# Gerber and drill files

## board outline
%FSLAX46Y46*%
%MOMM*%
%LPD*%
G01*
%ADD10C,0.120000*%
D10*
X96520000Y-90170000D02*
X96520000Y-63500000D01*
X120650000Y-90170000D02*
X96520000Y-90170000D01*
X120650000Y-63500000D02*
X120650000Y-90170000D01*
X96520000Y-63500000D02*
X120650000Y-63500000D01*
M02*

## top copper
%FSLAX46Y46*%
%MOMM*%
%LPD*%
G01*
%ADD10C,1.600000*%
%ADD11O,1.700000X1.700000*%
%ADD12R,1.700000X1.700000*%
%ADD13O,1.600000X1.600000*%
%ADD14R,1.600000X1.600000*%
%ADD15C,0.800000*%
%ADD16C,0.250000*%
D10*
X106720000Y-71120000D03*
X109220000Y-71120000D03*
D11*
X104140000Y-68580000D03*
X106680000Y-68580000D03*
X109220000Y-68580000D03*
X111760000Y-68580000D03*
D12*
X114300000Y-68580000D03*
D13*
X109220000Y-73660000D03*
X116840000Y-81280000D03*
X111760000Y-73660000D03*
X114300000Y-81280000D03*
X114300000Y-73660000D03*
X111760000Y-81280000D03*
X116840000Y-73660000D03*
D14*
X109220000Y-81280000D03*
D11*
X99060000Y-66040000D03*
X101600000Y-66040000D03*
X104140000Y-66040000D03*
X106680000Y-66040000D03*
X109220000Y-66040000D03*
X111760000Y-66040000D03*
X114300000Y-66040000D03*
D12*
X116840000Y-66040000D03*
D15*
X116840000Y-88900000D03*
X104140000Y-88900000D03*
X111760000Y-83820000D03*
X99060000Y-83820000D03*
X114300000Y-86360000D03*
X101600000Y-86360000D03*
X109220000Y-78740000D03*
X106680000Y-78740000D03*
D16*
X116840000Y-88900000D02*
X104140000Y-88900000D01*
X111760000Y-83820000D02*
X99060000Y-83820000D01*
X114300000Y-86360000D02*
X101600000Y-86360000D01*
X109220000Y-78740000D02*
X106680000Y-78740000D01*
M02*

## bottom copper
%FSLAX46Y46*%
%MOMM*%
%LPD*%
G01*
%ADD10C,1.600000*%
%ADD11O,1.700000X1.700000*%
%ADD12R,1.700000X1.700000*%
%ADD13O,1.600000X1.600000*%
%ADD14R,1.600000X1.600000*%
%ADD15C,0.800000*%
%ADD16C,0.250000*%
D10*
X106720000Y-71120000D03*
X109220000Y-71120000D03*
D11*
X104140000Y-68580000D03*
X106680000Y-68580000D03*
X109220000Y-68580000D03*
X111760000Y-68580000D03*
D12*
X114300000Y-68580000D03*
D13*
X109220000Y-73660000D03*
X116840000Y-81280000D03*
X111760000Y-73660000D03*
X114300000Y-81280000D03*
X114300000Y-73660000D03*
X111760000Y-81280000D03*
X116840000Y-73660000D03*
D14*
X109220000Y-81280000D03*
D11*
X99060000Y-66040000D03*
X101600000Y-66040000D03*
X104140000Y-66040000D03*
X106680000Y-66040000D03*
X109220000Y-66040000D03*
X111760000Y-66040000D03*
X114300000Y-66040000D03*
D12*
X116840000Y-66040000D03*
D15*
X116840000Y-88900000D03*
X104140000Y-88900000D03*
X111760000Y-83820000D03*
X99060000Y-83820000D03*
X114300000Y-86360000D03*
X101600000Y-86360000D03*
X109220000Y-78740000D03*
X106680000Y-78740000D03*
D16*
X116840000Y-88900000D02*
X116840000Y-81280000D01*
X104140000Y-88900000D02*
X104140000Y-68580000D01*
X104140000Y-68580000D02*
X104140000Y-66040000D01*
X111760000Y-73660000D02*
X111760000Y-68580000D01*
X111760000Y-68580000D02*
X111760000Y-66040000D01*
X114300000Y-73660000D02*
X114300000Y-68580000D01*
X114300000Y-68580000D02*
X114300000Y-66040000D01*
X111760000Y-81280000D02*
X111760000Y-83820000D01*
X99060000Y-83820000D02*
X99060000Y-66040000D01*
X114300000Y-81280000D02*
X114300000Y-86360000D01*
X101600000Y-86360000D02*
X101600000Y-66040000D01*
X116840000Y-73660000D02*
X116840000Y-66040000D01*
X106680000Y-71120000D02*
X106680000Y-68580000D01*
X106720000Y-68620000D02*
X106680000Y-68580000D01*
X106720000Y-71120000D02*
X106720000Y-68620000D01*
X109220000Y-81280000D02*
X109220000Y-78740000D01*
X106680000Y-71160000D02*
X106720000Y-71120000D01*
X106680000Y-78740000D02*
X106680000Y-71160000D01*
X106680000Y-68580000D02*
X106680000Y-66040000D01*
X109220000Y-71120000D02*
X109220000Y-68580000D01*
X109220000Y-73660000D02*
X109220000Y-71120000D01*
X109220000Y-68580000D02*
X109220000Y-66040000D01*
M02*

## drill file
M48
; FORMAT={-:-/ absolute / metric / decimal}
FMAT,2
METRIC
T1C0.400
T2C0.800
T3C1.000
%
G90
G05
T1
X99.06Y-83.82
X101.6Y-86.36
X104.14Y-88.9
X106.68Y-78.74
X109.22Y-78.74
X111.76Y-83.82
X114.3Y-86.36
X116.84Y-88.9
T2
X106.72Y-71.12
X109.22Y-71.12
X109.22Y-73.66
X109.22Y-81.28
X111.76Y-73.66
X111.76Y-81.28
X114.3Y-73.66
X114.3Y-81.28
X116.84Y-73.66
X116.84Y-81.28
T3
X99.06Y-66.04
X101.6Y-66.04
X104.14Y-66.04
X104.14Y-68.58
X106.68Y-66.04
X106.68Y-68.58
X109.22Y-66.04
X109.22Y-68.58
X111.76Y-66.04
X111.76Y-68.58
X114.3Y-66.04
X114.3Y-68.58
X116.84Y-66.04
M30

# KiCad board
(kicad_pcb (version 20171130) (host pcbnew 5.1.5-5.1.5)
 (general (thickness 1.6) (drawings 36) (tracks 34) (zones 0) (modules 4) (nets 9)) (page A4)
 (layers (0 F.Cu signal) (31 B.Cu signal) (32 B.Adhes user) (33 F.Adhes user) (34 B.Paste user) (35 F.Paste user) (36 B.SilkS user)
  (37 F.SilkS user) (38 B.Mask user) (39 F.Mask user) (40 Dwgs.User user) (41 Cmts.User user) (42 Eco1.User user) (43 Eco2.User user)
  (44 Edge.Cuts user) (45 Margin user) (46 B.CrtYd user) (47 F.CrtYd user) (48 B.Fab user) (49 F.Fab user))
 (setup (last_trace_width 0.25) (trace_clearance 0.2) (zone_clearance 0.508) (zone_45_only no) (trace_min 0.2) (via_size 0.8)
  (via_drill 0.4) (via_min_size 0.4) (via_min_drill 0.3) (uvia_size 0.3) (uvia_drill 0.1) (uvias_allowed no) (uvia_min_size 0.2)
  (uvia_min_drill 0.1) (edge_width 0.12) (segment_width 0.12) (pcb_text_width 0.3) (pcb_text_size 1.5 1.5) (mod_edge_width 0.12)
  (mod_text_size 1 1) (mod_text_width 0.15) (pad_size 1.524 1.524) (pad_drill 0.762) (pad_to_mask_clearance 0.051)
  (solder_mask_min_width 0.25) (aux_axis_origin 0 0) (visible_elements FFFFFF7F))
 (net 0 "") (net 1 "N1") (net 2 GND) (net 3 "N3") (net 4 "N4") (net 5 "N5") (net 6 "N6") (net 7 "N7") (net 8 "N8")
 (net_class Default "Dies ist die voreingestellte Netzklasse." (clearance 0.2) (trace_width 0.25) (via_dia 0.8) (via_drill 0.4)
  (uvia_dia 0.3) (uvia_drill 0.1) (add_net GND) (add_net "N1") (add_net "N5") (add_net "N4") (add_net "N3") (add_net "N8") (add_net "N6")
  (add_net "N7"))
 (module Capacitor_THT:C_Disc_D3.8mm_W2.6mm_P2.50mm (layer F.Cu) (at 109.22 71.12 180)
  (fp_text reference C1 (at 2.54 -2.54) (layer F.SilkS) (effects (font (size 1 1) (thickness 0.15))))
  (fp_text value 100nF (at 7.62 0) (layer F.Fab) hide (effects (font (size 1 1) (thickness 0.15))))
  (pad 2 thru_hole circle (at 2.5 0 180) (size 1.6 1.6) (drill 0.8) (layers *.Cu *.Mask) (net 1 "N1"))
  (pad 1 thru_hole circle (at 0 0 180) (size 1.6 1.6) (drill 0.8) (layers *.Cu *.Mask) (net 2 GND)))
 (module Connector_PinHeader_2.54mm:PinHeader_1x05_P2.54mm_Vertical (layer F.Cu) (at 114.3 68.58 270)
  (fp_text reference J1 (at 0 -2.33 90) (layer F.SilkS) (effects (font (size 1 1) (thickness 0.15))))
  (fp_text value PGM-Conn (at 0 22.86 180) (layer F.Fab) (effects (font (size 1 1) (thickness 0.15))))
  (pad 5 thru_hole oval (at 0 10.16 270) (size 1.7 1.7) (drill 1) (layers *.Cu *.Mask) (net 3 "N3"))
  (pad 4 thru_hole oval (at 0 7.62 270) (size 1.7 1.7) (drill 1) (layers *.Cu *.Mask) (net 1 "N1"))
  (pad 3 thru_hole oval (at 0 5.08 270) (size 1.7 1.7) (drill 1) (layers *.Cu *.Mask) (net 2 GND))
  (pad 2 thru_hole oval (at 0 2.54 270) (size 1.7 1.7) (drill 1) (layers *.Cu *.Mask) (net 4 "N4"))
  (pad 1 thru_hole rect (at 0 0 270) (size 1.7 1.7) (drill 1) (layers *.Cu *.Mask) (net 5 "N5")))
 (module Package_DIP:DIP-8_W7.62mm (layer F.Cu) (at 109.22 81.28 90)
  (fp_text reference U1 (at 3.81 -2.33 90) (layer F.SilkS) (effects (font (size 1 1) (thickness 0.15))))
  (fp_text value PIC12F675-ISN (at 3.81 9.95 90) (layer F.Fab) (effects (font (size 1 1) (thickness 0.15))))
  (pad 8 thru_hole oval (at 7.62 0 90) (size 1.6 1.6) (drill 0.8) (layers *.Cu *.Mask) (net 2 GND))
  (pad 4 thru_hole oval (at 0 7.62 90) (size 1.6 1.6) (drill 0.8) (layers *.Cu *.Mask) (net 3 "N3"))
  (pad 7 thru_hole oval (at 7.62 2.54 90) (size 1.6 1.6) (drill 0.8) (layers *.Cu *.Mask) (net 4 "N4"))
  (pad 3 thru_hole oval (at 0 5.08 90) (size 1.6 1.6) (drill 0.8) (layers *.Cu *.Mask) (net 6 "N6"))
  (pad 6 thru_hole oval (at 7.62 5.08 90) (size 1.6 1.6) (drill 0.8) (layers *.Cu *.Mask) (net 5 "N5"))
  (pad 2 thru_hole oval (at 0 2.54 90) (size 1.6 1.6) (drill 0.8) (layers *.Cu *.Mask) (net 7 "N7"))
  (pad 5 thru_hole oval (at 7.62 7.62 90) (size 1.6 1.6) (drill 0.8) (layers *.Cu *.Mask) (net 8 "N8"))
  (pad 1 thru_hole rect (at 0 0 90) (size 1.6 1.6) (drill 0.8) (layers *.Cu *.Mask) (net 1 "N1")))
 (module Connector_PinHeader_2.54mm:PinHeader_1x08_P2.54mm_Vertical (layer B.Cu) (at 116.84 66.04 90)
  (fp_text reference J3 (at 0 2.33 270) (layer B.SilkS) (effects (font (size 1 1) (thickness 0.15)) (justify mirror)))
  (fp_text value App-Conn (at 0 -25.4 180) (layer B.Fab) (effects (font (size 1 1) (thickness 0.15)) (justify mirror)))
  (pad 8 thru_hole oval (at 0 -17.78 90) (size 1.7 1.7) (drill 1) (layers *.Cu *.Mask) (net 7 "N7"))
  (pad 7 thru_hole oval (at 0 -15.24 90) (size 1.7 1.7) (drill 1) (layers *.Cu *.Mask) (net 6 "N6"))
  (pad 6 thru_hole oval (at 0 -12.7 90) (size 1.7 1.7) (drill 1) (layers *.Cu *.Mask) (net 3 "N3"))
  (pad 5 thru_hole oval (at 0 -10.16 90) (size 1.7 1.7) (drill 1) (layers *.Cu *.Mask) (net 1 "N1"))
  (pad 4 thru_hole oval (at 0 -7.62 90) (size 1.7 1.7) (drill 1) (layers *.Cu *.Mask) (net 2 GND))
  (pad 3 thru_hole oval (at 0 -5.08 90) (size 1.7 1.7) (drill 1) (layers *.Cu *.Mask) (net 4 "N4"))
  (pad 2 thru_hole oval (at 0 -2.54 90) (size 1.7 1.7) (drill 1) (layers *.Cu *.Mask) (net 5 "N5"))
  (pad 1 thru_hole rect (at 0 0 90) (size 1.7 1.7) (drill 1) (layers *.Cu *.Mask) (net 8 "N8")))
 (gr_line (start 96.52 90.17) (end 96.52 63.5) (layer Edge.Cuts) (width 0.12))
 (gr_line (start 120.65 90.17) (end 96.52 90.17) (layer Edge.Cuts) (width 0.12))
 (gr_line (start 120.65 63.5) (end 120.65 90.17) (layer Edge.Cuts) (width 0.12))
 (gr_line (start 96.52 63.5) (end 120.65 63.5) (layer Edge.Cuts) (width 0.12))
 (via (at 116.84 88.9) (size 0.8) (drill 0.4) (layers F.Cu B.Cu) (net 3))
 (via (at 104.14 88.9) (size 0.8) (drill 0.4) (layers F.Cu B.Cu) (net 3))
 (segment (start 116.84 88.9) (end 104.14 88.9) (width 0.25) (layer F.Cu) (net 3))
 (segment (start 116.84 88.9) (end 116.84 81.28) (width 0.25) (layer B.Cu) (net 3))
 (segment (start 104.14 88.9) (end 104.14 68.58) (width 0.25) (layer B.Cu) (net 3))
 (segment (start 104.14 68.58) (end 104.14 66.04) (width 0.25) (layer B.Cu) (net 3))
 (segment (start 111.76 73.66) (end 111.76 68.58) (width 0.25) (layer B.Cu) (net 4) (status 30))
 (segment (start 111.76 68.58) (end 111.76 66.04) (width 0.25) (layer B.Cu) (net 4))
 (segment (start 114.3 73.66) (end 114.3 68.58) (width 0.25) (layer B.Cu) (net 5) (status 30))
 (segment (start 114.3 68.58) (end 114.3 66.04) (width 0.25) (layer B.Cu) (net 5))
 (via (at 111.76 83.82) (size 0.8) (drill 0.4) (layers F.Cu B.Cu) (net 7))
 (segment (start 111.76 81.28) (end 111.76 83.82) (width 0.25) (layer B.Cu) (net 7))
 (via (at 99.06 83.82) (size 0.8) (drill 0.4) (layers F.Cu B.Cu) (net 7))
 (segment (start 111.76 83.82) (end 99.06 83.82) (width 0.25) (layer F.Cu) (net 7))
 (segment (start 99.06 83.82) (end 99.06 66.04) (width 0.25) (layer B.Cu) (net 7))
 (via (at 114.3 86.36) (size 0.8) (drill 0.4) (layers F.Cu B.Cu) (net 6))
 (segment (start 114.3 81.28) (end 114.3 86.36) (width 0.25) (layer B.Cu) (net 6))
 (via (at 101.6 86.36) (size 0.8) (drill 0.4) (layers F.Cu B.Cu) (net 6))
 (segment (start 114.3 86.36) (end 101.6 86.36) (width 0.25) (layer F.Cu) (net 6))
 (segment (start 101.6 86.36) (end 101.6 66.04) (width 0.25) (layer B.Cu) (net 6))
 (segment (start 116.84 73.66) (end 116.84 66.04) (width 0.25) (layer B.Cu) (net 8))
 (segment (start 106.68 71.12) (end 106.68 68.58) (width 0.25) (layer B.Cu) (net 1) (status 30))
 (segment (start 106.72 68.62) (end 106.68 68.58) (width 0.25) (layer B.Cu) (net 1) (status 30))
 (segment (start 106.72 71.12) (end 106.72 68.62) (width 0.25) (layer B.Cu) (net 1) (status 30))
 (via (at 109.22 78.74) (size 0.8) (drill 0.4) (layers F.Cu B.Cu) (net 1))
 (segment (start 109.22 81.28) (end 109.22 78.74) (width 0.25) (layer B.Cu) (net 1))
 (via (at 106.68 78.74) (size 0.8) (drill 0.4) (layers F.Cu B.Cu) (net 1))
 (segment (start 109.22 78.74) (end 106.68 78.74) (width 0.25) (layer F.Cu) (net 1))
 (segment (start 106.68 71.16) (end 106.72 71.12) (width 0.25) (layer B.Cu) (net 1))
 (segment (start 106.68 78.74) (end 106.68 71.16) (width 0.25) (layer B.Cu) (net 1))
 (segment (start 106.68 68.58) (end 106.68 66.04) (width 0.25) (layer B.Cu) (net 1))
 (segment (start 109.22 71.12) (end 109.22 68.58) (width 0.25) (layer B.Cu) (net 2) (status 30))
 (segment (start 109.22 73.66) (end 109.22 71.12) (width 0.25) (layer B.Cu) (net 2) (status 30))
 (segment (start 109.22 68.58) (end 109.22 66.04) (width 0.25) (layer B.Cu) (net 2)))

